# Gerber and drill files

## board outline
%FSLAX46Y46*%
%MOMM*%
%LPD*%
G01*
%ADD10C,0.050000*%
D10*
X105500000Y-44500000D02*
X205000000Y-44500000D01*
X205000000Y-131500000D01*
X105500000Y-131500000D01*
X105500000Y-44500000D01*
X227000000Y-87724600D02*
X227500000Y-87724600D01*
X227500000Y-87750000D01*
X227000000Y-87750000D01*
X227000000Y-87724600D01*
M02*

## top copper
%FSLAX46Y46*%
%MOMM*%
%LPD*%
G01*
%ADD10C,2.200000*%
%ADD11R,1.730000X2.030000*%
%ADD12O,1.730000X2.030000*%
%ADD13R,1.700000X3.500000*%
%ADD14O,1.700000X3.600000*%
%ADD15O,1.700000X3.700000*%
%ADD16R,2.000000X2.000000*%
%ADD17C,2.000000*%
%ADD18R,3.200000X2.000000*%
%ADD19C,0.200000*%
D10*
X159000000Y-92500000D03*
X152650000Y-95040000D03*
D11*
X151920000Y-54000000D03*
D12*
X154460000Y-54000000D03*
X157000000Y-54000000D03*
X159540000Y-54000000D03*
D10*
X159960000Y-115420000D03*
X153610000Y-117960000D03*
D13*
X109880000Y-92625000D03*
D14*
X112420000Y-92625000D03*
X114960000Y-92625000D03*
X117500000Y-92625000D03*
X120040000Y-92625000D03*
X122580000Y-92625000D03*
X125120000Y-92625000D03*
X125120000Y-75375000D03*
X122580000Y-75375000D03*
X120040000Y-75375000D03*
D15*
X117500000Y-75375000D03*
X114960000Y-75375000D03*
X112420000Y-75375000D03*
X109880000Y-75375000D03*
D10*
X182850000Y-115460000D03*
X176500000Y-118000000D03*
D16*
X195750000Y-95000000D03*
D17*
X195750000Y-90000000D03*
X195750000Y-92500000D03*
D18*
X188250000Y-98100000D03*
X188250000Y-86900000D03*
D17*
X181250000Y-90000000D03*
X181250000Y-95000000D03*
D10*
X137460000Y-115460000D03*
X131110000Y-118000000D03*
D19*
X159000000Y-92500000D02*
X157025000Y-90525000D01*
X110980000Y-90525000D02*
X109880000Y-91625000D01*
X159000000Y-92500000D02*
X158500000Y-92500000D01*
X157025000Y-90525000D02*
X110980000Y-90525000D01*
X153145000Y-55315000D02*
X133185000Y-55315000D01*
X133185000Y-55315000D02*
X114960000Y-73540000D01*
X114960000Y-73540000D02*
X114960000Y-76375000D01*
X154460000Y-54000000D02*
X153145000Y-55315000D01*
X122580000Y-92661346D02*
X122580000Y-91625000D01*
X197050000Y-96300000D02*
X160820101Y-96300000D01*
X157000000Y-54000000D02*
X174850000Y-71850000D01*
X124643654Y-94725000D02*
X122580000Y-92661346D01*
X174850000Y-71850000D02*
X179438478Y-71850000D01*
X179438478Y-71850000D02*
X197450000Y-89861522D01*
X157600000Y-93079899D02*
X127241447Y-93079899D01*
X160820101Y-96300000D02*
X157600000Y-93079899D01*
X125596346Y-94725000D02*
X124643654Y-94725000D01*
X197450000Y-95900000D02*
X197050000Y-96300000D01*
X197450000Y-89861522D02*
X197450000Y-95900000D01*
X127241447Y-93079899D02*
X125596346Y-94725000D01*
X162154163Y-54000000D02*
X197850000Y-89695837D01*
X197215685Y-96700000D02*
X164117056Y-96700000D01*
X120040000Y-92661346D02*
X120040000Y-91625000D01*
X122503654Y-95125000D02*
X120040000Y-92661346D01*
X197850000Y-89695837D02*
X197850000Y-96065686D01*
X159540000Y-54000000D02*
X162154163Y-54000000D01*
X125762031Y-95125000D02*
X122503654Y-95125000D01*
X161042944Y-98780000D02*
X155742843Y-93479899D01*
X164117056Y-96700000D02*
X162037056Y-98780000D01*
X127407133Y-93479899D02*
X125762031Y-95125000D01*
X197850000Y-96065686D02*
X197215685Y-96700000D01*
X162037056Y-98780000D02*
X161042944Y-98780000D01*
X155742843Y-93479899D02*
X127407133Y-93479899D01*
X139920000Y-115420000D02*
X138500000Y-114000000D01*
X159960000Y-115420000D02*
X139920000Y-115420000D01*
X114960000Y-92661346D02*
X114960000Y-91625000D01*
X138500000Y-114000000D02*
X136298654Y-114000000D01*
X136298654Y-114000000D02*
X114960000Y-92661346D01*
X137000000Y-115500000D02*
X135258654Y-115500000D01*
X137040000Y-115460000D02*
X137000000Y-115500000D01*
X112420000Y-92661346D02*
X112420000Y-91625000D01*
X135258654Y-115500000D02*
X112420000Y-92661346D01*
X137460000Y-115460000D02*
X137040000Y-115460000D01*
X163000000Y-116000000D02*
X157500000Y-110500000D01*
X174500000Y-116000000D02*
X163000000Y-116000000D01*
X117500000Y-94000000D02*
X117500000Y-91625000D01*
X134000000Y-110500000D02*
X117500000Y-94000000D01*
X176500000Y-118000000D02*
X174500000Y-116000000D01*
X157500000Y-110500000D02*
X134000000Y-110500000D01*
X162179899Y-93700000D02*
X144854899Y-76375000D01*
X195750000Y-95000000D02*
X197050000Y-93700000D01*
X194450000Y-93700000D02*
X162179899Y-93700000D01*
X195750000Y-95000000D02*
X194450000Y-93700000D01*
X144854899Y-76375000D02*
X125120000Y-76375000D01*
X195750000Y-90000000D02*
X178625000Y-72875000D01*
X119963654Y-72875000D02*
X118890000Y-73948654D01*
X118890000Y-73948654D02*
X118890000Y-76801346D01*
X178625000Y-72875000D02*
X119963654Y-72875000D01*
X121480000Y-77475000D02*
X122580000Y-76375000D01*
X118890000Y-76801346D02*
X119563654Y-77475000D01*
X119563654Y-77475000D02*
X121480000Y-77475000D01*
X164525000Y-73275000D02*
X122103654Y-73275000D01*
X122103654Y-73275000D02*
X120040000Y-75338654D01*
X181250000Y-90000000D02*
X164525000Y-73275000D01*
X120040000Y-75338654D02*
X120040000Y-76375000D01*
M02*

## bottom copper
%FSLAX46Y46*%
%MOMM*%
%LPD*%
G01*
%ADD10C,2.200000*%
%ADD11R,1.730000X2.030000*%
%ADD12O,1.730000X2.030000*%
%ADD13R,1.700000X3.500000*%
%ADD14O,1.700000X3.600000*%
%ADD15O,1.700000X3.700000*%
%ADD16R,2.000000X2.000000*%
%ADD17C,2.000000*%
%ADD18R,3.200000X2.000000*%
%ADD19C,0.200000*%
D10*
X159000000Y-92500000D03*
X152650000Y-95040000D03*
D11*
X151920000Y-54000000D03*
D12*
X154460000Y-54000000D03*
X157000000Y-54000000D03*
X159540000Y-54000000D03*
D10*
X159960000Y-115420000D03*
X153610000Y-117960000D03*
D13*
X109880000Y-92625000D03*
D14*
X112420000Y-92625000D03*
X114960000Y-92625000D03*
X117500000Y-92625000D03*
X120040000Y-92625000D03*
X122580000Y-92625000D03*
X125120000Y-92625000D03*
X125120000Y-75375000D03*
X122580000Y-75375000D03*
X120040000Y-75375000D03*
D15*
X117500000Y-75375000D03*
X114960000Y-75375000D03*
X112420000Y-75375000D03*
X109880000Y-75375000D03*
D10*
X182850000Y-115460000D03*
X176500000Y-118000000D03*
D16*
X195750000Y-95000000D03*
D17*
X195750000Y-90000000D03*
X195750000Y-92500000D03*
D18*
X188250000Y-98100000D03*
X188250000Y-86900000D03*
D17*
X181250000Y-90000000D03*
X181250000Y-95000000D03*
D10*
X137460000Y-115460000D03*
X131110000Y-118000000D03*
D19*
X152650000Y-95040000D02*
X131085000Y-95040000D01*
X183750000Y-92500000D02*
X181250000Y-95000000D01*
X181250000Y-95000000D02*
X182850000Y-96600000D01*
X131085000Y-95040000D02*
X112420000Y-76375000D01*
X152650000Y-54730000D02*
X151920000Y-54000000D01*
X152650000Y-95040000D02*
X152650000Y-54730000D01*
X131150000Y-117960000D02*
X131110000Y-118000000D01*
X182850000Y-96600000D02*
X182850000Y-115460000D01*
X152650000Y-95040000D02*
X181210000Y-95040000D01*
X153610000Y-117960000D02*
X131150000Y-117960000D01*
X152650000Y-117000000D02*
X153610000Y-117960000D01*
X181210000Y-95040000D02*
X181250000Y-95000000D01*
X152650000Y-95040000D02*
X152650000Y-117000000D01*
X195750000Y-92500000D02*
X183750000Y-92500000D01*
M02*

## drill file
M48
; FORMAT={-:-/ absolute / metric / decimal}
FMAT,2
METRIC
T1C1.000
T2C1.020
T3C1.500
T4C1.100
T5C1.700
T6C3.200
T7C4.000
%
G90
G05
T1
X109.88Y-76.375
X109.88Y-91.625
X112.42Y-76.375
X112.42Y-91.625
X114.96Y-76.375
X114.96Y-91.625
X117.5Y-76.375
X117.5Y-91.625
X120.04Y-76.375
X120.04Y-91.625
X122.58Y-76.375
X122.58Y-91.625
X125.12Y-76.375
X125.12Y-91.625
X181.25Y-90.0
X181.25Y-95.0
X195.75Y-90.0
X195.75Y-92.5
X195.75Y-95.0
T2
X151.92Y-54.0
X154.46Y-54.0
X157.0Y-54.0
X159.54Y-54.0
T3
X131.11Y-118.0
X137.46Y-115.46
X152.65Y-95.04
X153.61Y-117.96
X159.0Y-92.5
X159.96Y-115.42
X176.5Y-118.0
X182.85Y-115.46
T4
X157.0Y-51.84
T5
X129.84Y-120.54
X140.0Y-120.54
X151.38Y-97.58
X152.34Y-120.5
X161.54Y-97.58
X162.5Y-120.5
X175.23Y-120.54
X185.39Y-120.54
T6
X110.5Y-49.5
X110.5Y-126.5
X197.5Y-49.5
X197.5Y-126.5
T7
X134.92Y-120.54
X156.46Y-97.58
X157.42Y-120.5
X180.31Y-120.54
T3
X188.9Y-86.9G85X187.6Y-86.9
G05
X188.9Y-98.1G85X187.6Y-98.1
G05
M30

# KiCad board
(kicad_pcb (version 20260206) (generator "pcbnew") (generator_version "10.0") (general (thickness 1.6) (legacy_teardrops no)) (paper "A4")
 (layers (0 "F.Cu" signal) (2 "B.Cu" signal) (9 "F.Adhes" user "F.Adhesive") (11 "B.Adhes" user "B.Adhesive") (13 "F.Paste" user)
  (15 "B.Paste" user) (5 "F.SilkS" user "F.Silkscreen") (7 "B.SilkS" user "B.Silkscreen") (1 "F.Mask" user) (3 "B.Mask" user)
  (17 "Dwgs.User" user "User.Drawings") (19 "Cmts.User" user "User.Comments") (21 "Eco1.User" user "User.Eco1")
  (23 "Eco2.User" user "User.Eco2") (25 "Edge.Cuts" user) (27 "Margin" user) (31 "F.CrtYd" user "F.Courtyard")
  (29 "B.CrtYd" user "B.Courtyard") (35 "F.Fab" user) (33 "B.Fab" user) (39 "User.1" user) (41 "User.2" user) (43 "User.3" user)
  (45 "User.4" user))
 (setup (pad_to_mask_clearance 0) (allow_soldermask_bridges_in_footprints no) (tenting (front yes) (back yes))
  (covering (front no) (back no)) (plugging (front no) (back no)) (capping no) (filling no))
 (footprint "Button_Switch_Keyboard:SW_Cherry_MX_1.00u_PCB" (layer "F.Cu") (at 159 92.5)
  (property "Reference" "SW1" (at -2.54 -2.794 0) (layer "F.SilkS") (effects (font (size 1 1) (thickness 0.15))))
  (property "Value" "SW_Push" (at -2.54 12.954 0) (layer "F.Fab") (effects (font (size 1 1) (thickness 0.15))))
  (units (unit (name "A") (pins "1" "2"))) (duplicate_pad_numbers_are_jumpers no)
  (pad "" np_thru_hole circle (at -7.62 5.08) (size 1.7 1.7) (drill 1.7) (layers "*.Cu" "*.Mask"))
  (pad "" np_thru_hole circle (at -2.54 5.08) (size 4 4) (drill 4) (layers "*.Cu" "*.Mask"))
  (pad "" np_thru_hole circle (at 2.54 5.08) (size 1.7 1.7) (drill 1.7) (layers "*.Cu" "*.Mask"))
  (pad "1" thru_hole circle (at 0 0) (size 2.2 2.2) (drill 1.5) (layers "*.Cu" "*.Mask") (remove_unused_layers no)
   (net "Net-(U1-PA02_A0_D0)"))
  (pad "2" thru_hole circle (at -6.35 2.54) (size 2.2 2.2) (drill 1.5) (layers "*.Cu" "*.Mask") (remove_unused_layers no) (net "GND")))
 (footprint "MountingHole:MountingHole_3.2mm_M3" (layer "F.Cu") (at 110.5 49.5)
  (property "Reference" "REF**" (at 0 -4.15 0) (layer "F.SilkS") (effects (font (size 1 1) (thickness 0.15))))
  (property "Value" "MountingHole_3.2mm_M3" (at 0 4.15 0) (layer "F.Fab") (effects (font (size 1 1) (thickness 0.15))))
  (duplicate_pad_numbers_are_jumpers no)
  (pad "" np_thru_hole circle (at 0 0) (size 3.2 3.2) (drill 3.2) (layers "*.Cu" "*.Mask")))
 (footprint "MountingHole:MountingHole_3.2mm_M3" (layer "F.Cu") (at 110.5 126.5)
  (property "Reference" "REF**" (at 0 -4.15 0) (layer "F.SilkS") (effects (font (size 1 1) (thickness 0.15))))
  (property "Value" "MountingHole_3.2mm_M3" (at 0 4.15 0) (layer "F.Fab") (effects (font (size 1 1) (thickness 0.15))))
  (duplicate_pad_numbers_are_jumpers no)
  (pad "" np_thru_hole circle (at 0 0) (size 3.2 3.2) (drill 3.2) (layers "*.Cu" "*.Mask")))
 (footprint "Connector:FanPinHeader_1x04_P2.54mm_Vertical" (layer "F.Cu") (at 151.92 54)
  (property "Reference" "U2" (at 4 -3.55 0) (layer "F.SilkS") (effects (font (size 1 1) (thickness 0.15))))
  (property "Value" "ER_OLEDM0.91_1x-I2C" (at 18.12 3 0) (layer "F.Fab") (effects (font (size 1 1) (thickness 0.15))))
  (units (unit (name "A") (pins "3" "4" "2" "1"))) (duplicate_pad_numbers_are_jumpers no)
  (pad "" np_thru_hole circle (at 5.08 -2.16 90) (size 1.1 1.1) (drill 1.1) (layers "*.Cu" "*.Mask"))
  (pad "1" thru_hole rect (at 0 0 90) (size 2.03 1.73) (drill 1.02) (layers "*.Cu" "*.Mask") (remove_unused_layers no) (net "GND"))
  (pad "2" thru_hole oval (at 2.54 0 90) (size 2.03 1.73) (drill 1.02) (layers "*.Cu" "*.Mask") (remove_unused_layers no)
   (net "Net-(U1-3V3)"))
  (pad "3" thru_hole oval (at 5.08 0 90) (size 2.03 1.73) (drill 1.02) (layers "*.Cu" "*.Mask") (remove_unused_layers no)
   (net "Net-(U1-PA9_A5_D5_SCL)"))
  (pad "4" thru_hole oval (at 7.62 0 90) (size 2.03 1.73) (drill 1.02) (layers "*.Cu" "*.Mask") (remove_unused_layers no)
   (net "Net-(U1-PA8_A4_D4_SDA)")))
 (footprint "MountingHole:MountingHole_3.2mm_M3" (layer "F.Cu") (at 197.5 126.5)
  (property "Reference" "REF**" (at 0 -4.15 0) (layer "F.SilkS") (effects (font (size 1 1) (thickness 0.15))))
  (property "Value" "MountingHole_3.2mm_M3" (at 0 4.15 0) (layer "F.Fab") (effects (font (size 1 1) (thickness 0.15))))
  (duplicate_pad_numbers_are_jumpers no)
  (pad "" np_thru_hole circle (at 0 0) (size 3.2 3.2) (drill 3.2) (layers "*.Cu" "*.Mask")))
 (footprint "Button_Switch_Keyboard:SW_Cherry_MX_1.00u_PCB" (layer "F.Cu") (at 159.96 115.42)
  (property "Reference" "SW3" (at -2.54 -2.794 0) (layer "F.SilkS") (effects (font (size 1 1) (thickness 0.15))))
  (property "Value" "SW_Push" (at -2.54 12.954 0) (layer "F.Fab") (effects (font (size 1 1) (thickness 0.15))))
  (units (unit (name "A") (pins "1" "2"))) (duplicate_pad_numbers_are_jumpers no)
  (pad "" np_thru_hole circle (at -7.62 5.08) (size 1.7 1.7) (drill 1.7) (layers "*.Cu" "*.Mask"))
  (pad "" np_thru_hole circle (at -2.54 5.08) (size 4 4) (drill 4) (layers "*.Cu" "*.Mask"))
  (pad "" np_thru_hole circle (at 2.54 5.08) (size 1.7 1.7) (drill 1.7) (layers "*.Cu" "*.Mask"))
  (pad "1" thru_hole circle (at 0 0) (size 2.2 2.2) (drill 1.5) (layers "*.Cu" "*.Mask") (remove_unused_layers no)
   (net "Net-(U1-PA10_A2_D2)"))
  (pad "2" thru_hole circle (at -6.35 2.54) (size 2.2 2.2) (drill 1.5) (layers "*.Cu" "*.Mask") (remove_unused_layers no) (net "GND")))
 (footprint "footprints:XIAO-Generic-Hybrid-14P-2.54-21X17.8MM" (layer "F.Cu") (at 117.5 84 90)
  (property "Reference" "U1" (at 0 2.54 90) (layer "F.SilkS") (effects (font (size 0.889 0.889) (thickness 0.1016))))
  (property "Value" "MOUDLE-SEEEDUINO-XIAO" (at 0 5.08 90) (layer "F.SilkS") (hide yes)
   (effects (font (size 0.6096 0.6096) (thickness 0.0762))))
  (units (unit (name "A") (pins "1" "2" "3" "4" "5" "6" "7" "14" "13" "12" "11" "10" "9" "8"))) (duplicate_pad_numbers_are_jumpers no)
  (pad "1" thru_hole rect (at -7.625 -7.62 90) (size 3.5 1.7) (drill 1 (offset -1 0)) (layers "*.Cu" "*.Mask") (remove_unused_layers no)
   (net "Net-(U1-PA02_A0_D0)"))
  (pad "2" thru_hole oval (at -7.625 -5.08 90) (size 3.6 1.7) (drill 1 (offset -1 0)) (layers "*.Cu" "*.Mask") (remove_unused_layers no)
   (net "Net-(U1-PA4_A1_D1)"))
  (pad "3" thru_hole oval (at -7.625 -2.54 90) (size 3.6 1.7) (drill 1 (offset -1 0)) (layers "*.Cu" "*.Mask") (remove_unused_layers no)
   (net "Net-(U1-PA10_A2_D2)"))
  (pad "4" thru_hole oval (at -7.625 0 90) (size 3.6 1.7) (drill 1 (offset -1 0)) (layers "*.Cu" "*.Mask") (remove_unused_layers no)
   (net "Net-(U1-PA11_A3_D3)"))
  (pad "5" thru_hole oval (at -7.625 2.54 90) (size 3.6 1.7) (drill 1 (offset -1 0)) (layers "*.Cu" "*.Mask") (remove_unused_layers no)
   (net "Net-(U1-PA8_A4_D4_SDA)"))
  (pad "6" thru_hole oval (at -7.625 5.08 270) (size 3.6 1.7) (drill 1 (offset 1 0)) (layers "*.Cu" "*.Mask") (remove_unused_layers no)
   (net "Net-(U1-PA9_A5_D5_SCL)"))
  (pad "7" thru_hole oval (at -7.625 7.62 90) (size 3.6 1.7) (drill 1 (offset -1 0)) (layers "*.Cu" "*.Mask") (remove_unused_layers no)
   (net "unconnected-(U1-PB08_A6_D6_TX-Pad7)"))
  (pad "8" thru_hole oval (at 7.625 7.62 90) (size 3.6 1.7) (drill 1 (offset 1 0)) (layers "*.Cu" "*.Mask") (remove_unused_layers no)
   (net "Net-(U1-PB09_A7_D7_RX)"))
  (pad "9" thru_hole oval (at 7.625 5.08 90) (size 3.6 1.7) (drill 1 (offset 1 0)) (layers "*.Cu" "*.Mask") (remove_unused_layers no)
   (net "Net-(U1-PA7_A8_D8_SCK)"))
  (pad "10" thru_hole oval (at 7.625 2.54 90) (size 3.6 1.7) (drill 1 (offset 1 0)) (layers "*.Cu" "*.Mask") (remove_unused_layers no)
   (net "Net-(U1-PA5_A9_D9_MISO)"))
  (pad "11" thru_hole oval (at 7.625 0 90) (size 3.7 1.7) (drill 1 (offset 1 0)) (layers "*.Cu" "*.Mask") (remove_unused_layers no)
   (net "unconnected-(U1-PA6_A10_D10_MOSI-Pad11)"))
  (pad "12" thru_hole oval (at 7.625 -2.54 90) (size 3.7 1.7) (drill 1 (offset 1 0)) (layers "*.Cu" "*.Mask") (remove_unused_layers no)
   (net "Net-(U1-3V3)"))
  (pad "13" thru_hole oval (at 7.625 -5.08 90) (size 3.7 1.7) (drill 1 (offset 1 0)) (layers "*.Cu" "*.Mask") (remove_unused_layers no)
   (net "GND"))
  (pad "14" thru_hole oval (at 7.625 -7.62 90) (size 3.7 1.7) (drill 1 (offset 1 0)) (layers "*.Cu" "*.Mask") (remove_unused_layers no)
   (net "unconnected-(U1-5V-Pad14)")))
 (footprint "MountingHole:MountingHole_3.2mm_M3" (layer "F.Cu") (at 197.5 49.5)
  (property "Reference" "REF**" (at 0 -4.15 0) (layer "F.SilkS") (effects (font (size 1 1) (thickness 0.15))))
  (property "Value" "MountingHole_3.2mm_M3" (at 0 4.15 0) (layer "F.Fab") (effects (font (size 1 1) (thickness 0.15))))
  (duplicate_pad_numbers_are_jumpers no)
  (pad "" np_thru_hole circle (at 0 0) (size 3.2 3.2) (drill 3.2) (layers "*.Cu" "*.Mask")))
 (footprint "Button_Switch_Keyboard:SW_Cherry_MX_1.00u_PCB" (layer "F.Cu") (at 182.85 115.46)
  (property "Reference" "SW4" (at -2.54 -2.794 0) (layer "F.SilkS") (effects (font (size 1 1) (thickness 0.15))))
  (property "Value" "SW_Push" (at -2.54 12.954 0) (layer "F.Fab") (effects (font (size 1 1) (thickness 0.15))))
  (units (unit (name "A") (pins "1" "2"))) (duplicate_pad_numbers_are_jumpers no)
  (pad "" np_thru_hole circle (at -7.62 5.08) (size 1.7 1.7) (drill 1.7) (layers "*.Cu" "*.Mask"))
  (pad "" np_thru_hole circle (at -2.54 5.08) (size 4 4) (drill 4) (layers "*.Cu" "*.Mask"))
  (pad "" np_thru_hole circle (at 2.54 5.08) (size 1.7 1.7) (drill 1.7) (layers "*.Cu" "*.Mask"))
  (pad "1" thru_hole circle (at 0 0) (size 2.2 2.2) (drill 1.5) (layers "*.Cu" "*.Mask") (remove_unused_layers no) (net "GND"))
  (pad "2" thru_hole circle (at -6.35 2.54) (size 2.2 2.2) (drill 1.5) (layers "*.Cu" "*.Mask") (remove_unused_layers no)
   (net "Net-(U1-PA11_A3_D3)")))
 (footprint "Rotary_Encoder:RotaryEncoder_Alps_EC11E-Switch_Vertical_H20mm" (layer "F.Cu") (at 195.75 95 180)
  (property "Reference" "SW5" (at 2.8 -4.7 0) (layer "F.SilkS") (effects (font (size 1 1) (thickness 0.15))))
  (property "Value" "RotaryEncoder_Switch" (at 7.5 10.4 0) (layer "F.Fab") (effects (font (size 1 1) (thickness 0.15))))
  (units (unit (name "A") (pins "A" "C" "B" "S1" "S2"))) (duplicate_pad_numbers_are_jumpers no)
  (pad "A" thru_hole rect (at 0 0 180) (size 2 2) (drill 1) (layers "*.Cu" "*.Mask") (remove_unused_layers no)
   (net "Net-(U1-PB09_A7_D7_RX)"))
  (pad "B" thru_hole circle (at 0 5 180) (size 2 2) (drill 1) (layers "*.Cu" "*.Mask") (remove_unused_layers no)
   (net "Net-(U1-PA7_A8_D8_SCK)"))
  (pad "C" thru_hole circle (at 0 2.5 180) (size 2 2) (drill 1) (layers "*.Cu" "*.Mask") (remove_unused_layers no) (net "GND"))
  (pad "MP" thru_hole rect (at 7.5 -3.1 180) (size 3.2 2) (drill oval 2.8 1.5) (layers "*.Cu" "*.Mask") (remove_unused_layers no))
  (pad "MP" thru_hole rect (at 7.5 8.1 180) (size 3.2 2) (drill oval 2.8 1.5) (layers "*.Cu" "*.Mask") (remove_unused_layers no))
  (pad "S1" thru_hole circle (at 14.5 5 180) (size 2 2) (drill 1) (layers "*.Cu" "*.Mask") (remove_unused_layers no)
   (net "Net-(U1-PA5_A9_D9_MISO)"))
  (pad "S2" thru_hole circle (at 14.5 0 180) (size 2 2) (drill 1) (layers "*.Cu" "*.Mask") (remove_unused_layers no) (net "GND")))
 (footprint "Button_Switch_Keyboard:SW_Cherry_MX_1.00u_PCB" (layer "F.Cu") (at 137.46 115.46)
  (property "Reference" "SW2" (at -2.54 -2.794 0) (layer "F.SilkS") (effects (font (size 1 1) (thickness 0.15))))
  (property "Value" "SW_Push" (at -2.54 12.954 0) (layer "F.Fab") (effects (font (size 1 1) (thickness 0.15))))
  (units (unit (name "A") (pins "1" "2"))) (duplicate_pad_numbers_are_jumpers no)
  (pad "" np_thru_hole circle (at -7.62 5.08) (size 1.7 1.7) (drill 1.7) (layers "*.Cu" "*.Mask"))
  (pad "" np_thru_hole circle (at -2.54 5.08) (size 4 4) (drill 4) (layers "*.Cu" "*.Mask"))
  (pad "" np_thru_hole circle (at 2.54 5.08) (size 1.7 1.7) (drill 1.7) (layers "*.Cu" "*.Mask"))
  (pad "1" thru_hole circle (at 0 0) (size 2.2 2.2) (drill 1.5) (layers "*.Cu" "*.Mask") (remove_unused_layers no)
   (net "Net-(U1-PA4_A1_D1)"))
  (pad "2" thru_hole circle (at -6.35 2.54) (size 2.2 2.2) (drill 1.5) (layers "*.Cu" "*.Mask") (remove_unused_layers no) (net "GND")))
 (gr_rect (start 105.5 44.5) (end 205 131.5) (stroke (width 0.05) (type default)) (fill no) (layer "Edge.Cuts"))
 (gr_rect (start 227 87.7246) (end 227.5 87.75) (stroke (width 0.05) (type default)) (fill no) (layer "Edge.Cuts"))
 (segment (start 159 92.5) (end 157.025 90.525) (width 0.2) (layer "F.Cu") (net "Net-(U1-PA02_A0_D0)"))
 (segment (start 110.98 90.525) (end 109.88 91.625) (width 0.2) (layer "F.Cu") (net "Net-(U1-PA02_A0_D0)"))
 (segment (start 159 92.5) (end 158.5 92.5) (width 0.2) (layer "F.Cu") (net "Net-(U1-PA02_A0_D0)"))
 (segment (start 157.025 90.525) (end 110.98 90.525) (width 0.2) (layer "F.Cu") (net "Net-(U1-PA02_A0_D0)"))
 (segment (start 152.65 95.04) (end 131.085 95.04) (width 0.2) (layer "B.Cu") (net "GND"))
 (segment (start 183.75 92.5) (end 181.25 95) (width 0.2) (layer "B.Cu") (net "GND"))
 (segment (start 181.25 95) (end 182.85 96.6) (width 0.2) (layer "B.Cu") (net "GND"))
 (segment (start 131.085 95.04) (end 112.42 76.375) (width 0.2) (layer "B.Cu") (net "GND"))
 (segment (start 152.65 54.73) (end 151.92 54) (width 0.2) (layer "B.Cu") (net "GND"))
 (segment (start 152.65 95.04) (end 152.65 54.73) (width 0.2) (layer "B.Cu") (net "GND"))
 (segment (start 131.15 117.96) (end 131.11 118) (width 0.2) (layer "B.Cu") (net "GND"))
 (segment (start 182.85 96.6) (end 182.85 115.46) (width 0.2) (layer "B.Cu") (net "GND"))
 (segment (start 152.65 95.04) (end 181.21 95.04) (width 0.2) (layer "B.Cu") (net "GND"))
 (segment (start 153.61 117.96) (end 131.15 117.96) (width 0.2) (layer "B.Cu") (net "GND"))
 (segment (start 152.65 117) (end 153.61 117.96) (width 0.2) (layer "B.Cu") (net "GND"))
 (segment (start 181.21 95.04) (end 181.25 95) (width 0.2) (layer "B.Cu") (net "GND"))
 (segment (start 152.65 95.04) (end 152.65 117) (width 0.2) (layer "B.Cu") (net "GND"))
 (segment (start 195.75 92.5) (end 183.75 92.5) (width 0.2) (layer "B.Cu") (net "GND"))
 (segment (start 153.145 55.315) (end 133.185 55.315) (width 0.2) (layer "F.Cu") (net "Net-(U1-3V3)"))
 (segment (start 133.185 55.315) (end 114.96 73.54) (width 0.2) (layer "F.Cu") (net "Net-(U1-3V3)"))
 (segment (start 114.96 73.54) (end 114.96 76.375) (width 0.2) (layer "F.Cu") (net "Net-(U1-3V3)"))
 (segment (start 154.46 54) (end 153.145 55.315) (width 0.2) (layer "F.Cu") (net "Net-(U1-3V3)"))
 (segment (start 122.58 92.661346) (end 122.58 91.625) (width 0.2) (layer "F.Cu") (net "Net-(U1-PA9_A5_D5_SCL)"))
 (segment (start 197.05 96.3) (end 160.820101 96.3) (width 0.2) (layer "F.Cu") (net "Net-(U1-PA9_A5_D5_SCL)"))
 (segment (start 157 54) (end 174.85 71.85) (width 0.2) (layer "F.Cu") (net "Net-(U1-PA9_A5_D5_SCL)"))
 (segment (start 124.643654 94.725) (end 122.58 92.661346) (width 0.2) (layer "F.Cu") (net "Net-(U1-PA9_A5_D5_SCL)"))
 (segment (start 174.85 71.85) (end 179.438478 71.85) (width 0.2) (layer "F.Cu") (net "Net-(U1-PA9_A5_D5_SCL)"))
 (segment (start 179.438478 71.85) (end 197.45 89.861522) (width 0.2) (layer "F.Cu") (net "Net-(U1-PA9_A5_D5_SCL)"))
 (segment (start 157.6 93.079899) (end 127.241447 93.079899) (width 0.2) (layer "F.Cu") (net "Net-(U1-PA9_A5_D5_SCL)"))
 (segment (start 160.820101 96.3) (end 157.6 93.079899) (width 0.2) (layer "F.Cu") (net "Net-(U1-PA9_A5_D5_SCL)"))
 (segment (start 125.596346 94.725) (end 124.643654 94.725) (width 0.2) (layer "F.Cu") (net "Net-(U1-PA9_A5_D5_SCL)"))
 (segment (start 197.45 95.9) (end 197.05 96.3) (width 0.2) (layer "F.Cu") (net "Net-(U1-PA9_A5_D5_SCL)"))
 (segment (start 197.45 89.861522) (end 197.45 95.9) (width 0.2) (layer "F.Cu") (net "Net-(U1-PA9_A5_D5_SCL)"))
 (segment (start 127.241447 93.079899) (end 125.596346 94.725) (width 0.2) (layer "F.Cu") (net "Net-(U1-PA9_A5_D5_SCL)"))
 (segment (start 162.154163 54) (end 197.85 89.695837) (width 0.2) (layer "F.Cu") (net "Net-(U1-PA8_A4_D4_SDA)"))
 (segment (start 197.215685 96.7) (end 164.117056 96.7) (width 0.2) (layer "F.Cu") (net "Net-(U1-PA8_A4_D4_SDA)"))
 (segment (start 120.04 92.661346) (end 120.04 91.625) (width 0.2) (layer "F.Cu") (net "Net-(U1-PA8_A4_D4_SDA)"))
 (segment (start 122.503654 95.125) (end 120.04 92.661346) (width 0.2) (layer "F.Cu") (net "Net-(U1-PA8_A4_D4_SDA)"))
 (segment (start 197.85 89.695837) (end 197.85 96.065686) (width 0.2) (layer "F.Cu") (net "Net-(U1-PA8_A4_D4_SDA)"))
 (segment (start 159.54 54) (end 162.154163 54) (width 0.2) (layer "F.Cu") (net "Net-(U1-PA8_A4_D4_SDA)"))
 (segment (start 125.762031 95.125) (end 122.503654 95.125) (width 0.2) (layer "F.Cu") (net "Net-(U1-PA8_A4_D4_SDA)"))
 (segment (start 161.042944 98.78) (end 155.742843 93.479899) (width 0.2) (layer "F.Cu") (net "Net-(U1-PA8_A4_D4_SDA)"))
 (segment (start 164.117056 96.7) (end 162.037056 98.78) (width 0.2) (layer "F.Cu") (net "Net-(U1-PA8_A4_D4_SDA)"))
 (segment (start 127.407133 93.479899) (end 125.762031 95.125) (width 0.2) (layer "F.Cu") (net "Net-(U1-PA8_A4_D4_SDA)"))
 (segment (start 197.85 96.065686) (end 197.215685 96.7) (width 0.2) (layer "F.Cu") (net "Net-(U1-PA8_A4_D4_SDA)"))
 (segment (start 162.037056 98.78) (end 161.042944 98.78) (width 0.2) (layer "F.Cu") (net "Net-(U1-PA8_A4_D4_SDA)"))
 (segment (start 155.742843 93.479899) (end 127.407133 93.479899) (width 0.2) (layer "F.Cu") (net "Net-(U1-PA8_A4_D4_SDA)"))
 (segment (start 139.92 115.42) (end 138.5 114) (width 0.2) (layer "F.Cu") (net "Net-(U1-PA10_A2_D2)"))
 (segment (start 159.96 115.42) (end 139.92 115.42) (width 0.2) (layer "F.Cu") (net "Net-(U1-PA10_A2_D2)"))
 (segment (start 114.96 92.661346) (end 114.96 91.625) (width 0.2) (layer "F.Cu") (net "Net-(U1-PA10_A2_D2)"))
 (segment (start 138.5 114) (end 136.298654 114) (width 0.2) (layer "F.Cu") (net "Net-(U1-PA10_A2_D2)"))
 (segment (start 136.298654 114) (end 114.96 92.661346) (width 0.2) (layer "F.Cu") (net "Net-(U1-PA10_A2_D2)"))
 (segment (start 137 115.5) (end 135.258654 115.5) (width 0.2) (layer "F.Cu") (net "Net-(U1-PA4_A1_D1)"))
 (segment (start 137.04 115.46) (end 137 115.5) (width 0.2) (layer "F.Cu") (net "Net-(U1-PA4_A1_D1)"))
 (segment (start 112.42 92.661346) (end 112.42 91.625) (width 0.2) (layer "F.Cu") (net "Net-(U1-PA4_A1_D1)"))
 (segment (start 135.258654 115.5) (end 112.42 92.661346) (width 0.2) (layer "F.Cu") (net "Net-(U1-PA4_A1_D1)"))
 (segment (start 137.46 115.46) (end 137.04 115.46) (width 0.2) (layer "F.Cu") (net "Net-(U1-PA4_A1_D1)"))
 (segment (start 163 116) (end 157.5 110.5) (width 0.2) (layer "F.Cu") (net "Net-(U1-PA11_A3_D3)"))
 (segment (start 174.5 116) (end 163 116) (width 0.2) (layer "F.Cu") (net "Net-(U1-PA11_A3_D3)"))
 (segment (start 117.5 94) (end 117.5 91.625) (width 0.2) (layer "F.Cu") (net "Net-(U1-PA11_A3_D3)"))
 (segment (start 134 110.5) (end 117.5 94) (width 0.2) (layer "F.Cu") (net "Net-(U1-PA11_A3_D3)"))
 (segment (start 176.5 118) (end 174.5 116) (width 0.2) (layer "F.Cu") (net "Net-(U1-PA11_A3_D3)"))
 (segment (start 157.5 110.5) (end 134 110.5) (width 0.2) (layer "F.Cu") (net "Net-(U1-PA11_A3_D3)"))
 (segment (start 162.179899 93.7) (end 144.854899 76.375) (width 0.2) (layer "F.Cu") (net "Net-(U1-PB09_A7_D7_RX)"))
 (segment (start 195.75 95) (end 197.05 93.7) (width 0.2) (layer "F.Cu") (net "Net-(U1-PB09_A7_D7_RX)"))
 (segment (start 194.45 93.7) (end 162.179899 93.7) (width 0.2) (layer "F.Cu") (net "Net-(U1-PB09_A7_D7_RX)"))
 (segment (start 195.75 95) (end 194.45 93.7) (width 0.2) (layer "F.Cu") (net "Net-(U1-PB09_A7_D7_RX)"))
 (segment (start 144.854899 76.375) (end 125.12 76.375) (width 0.2) (layer "F.Cu") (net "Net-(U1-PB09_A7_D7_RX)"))
 (segment (start 195.75 90) (end 178.625 72.875) (width 0.2) (layer "F.Cu") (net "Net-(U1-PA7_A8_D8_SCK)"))
 (segment (start 119.963654 72.875) (end 118.89 73.948654) (width 0.2) (layer "F.Cu") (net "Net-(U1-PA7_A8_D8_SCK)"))
 (segment (start 118.89 73.948654) (end 118.89 76.801346) (width 0.2) (layer "F.Cu") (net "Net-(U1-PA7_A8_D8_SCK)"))
 (segment (start 178.625 72.875) (end 119.963654 72.875) (width 0.2) (layer "F.Cu") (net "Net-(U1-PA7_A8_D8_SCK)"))
 (segment (start 121.48 77.475) (end 122.58 76.375) (width 0.2) (layer "F.Cu") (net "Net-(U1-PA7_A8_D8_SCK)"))
 (segment (start 118.89 76.801346) (end 119.563654 77.475) (width 0.2) (layer "F.Cu") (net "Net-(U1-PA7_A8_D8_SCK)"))
 (segment (start 119.563654 77.475) (end 121.48 77.475) (width 0.2) (layer "F.Cu") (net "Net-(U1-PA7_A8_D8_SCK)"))
 (segment (start 164.525 73.275) (end 122.103654 73.275) (width 0.2) (layer "F.Cu") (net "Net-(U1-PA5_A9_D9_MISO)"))
 (segment (start 122.103654 73.275) (end 120.04 75.338654) (width 0.2) (layer "F.Cu") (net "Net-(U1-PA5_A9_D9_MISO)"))
 (segment (start 181.25 90) (end 164.525 73.275) (width 0.2) (layer "F.Cu") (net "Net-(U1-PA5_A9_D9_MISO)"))
 (segment (start 120.04 75.338654) (end 120.04 76.375) (width 0.2) (layer "F.Cu") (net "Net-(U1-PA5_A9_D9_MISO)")))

